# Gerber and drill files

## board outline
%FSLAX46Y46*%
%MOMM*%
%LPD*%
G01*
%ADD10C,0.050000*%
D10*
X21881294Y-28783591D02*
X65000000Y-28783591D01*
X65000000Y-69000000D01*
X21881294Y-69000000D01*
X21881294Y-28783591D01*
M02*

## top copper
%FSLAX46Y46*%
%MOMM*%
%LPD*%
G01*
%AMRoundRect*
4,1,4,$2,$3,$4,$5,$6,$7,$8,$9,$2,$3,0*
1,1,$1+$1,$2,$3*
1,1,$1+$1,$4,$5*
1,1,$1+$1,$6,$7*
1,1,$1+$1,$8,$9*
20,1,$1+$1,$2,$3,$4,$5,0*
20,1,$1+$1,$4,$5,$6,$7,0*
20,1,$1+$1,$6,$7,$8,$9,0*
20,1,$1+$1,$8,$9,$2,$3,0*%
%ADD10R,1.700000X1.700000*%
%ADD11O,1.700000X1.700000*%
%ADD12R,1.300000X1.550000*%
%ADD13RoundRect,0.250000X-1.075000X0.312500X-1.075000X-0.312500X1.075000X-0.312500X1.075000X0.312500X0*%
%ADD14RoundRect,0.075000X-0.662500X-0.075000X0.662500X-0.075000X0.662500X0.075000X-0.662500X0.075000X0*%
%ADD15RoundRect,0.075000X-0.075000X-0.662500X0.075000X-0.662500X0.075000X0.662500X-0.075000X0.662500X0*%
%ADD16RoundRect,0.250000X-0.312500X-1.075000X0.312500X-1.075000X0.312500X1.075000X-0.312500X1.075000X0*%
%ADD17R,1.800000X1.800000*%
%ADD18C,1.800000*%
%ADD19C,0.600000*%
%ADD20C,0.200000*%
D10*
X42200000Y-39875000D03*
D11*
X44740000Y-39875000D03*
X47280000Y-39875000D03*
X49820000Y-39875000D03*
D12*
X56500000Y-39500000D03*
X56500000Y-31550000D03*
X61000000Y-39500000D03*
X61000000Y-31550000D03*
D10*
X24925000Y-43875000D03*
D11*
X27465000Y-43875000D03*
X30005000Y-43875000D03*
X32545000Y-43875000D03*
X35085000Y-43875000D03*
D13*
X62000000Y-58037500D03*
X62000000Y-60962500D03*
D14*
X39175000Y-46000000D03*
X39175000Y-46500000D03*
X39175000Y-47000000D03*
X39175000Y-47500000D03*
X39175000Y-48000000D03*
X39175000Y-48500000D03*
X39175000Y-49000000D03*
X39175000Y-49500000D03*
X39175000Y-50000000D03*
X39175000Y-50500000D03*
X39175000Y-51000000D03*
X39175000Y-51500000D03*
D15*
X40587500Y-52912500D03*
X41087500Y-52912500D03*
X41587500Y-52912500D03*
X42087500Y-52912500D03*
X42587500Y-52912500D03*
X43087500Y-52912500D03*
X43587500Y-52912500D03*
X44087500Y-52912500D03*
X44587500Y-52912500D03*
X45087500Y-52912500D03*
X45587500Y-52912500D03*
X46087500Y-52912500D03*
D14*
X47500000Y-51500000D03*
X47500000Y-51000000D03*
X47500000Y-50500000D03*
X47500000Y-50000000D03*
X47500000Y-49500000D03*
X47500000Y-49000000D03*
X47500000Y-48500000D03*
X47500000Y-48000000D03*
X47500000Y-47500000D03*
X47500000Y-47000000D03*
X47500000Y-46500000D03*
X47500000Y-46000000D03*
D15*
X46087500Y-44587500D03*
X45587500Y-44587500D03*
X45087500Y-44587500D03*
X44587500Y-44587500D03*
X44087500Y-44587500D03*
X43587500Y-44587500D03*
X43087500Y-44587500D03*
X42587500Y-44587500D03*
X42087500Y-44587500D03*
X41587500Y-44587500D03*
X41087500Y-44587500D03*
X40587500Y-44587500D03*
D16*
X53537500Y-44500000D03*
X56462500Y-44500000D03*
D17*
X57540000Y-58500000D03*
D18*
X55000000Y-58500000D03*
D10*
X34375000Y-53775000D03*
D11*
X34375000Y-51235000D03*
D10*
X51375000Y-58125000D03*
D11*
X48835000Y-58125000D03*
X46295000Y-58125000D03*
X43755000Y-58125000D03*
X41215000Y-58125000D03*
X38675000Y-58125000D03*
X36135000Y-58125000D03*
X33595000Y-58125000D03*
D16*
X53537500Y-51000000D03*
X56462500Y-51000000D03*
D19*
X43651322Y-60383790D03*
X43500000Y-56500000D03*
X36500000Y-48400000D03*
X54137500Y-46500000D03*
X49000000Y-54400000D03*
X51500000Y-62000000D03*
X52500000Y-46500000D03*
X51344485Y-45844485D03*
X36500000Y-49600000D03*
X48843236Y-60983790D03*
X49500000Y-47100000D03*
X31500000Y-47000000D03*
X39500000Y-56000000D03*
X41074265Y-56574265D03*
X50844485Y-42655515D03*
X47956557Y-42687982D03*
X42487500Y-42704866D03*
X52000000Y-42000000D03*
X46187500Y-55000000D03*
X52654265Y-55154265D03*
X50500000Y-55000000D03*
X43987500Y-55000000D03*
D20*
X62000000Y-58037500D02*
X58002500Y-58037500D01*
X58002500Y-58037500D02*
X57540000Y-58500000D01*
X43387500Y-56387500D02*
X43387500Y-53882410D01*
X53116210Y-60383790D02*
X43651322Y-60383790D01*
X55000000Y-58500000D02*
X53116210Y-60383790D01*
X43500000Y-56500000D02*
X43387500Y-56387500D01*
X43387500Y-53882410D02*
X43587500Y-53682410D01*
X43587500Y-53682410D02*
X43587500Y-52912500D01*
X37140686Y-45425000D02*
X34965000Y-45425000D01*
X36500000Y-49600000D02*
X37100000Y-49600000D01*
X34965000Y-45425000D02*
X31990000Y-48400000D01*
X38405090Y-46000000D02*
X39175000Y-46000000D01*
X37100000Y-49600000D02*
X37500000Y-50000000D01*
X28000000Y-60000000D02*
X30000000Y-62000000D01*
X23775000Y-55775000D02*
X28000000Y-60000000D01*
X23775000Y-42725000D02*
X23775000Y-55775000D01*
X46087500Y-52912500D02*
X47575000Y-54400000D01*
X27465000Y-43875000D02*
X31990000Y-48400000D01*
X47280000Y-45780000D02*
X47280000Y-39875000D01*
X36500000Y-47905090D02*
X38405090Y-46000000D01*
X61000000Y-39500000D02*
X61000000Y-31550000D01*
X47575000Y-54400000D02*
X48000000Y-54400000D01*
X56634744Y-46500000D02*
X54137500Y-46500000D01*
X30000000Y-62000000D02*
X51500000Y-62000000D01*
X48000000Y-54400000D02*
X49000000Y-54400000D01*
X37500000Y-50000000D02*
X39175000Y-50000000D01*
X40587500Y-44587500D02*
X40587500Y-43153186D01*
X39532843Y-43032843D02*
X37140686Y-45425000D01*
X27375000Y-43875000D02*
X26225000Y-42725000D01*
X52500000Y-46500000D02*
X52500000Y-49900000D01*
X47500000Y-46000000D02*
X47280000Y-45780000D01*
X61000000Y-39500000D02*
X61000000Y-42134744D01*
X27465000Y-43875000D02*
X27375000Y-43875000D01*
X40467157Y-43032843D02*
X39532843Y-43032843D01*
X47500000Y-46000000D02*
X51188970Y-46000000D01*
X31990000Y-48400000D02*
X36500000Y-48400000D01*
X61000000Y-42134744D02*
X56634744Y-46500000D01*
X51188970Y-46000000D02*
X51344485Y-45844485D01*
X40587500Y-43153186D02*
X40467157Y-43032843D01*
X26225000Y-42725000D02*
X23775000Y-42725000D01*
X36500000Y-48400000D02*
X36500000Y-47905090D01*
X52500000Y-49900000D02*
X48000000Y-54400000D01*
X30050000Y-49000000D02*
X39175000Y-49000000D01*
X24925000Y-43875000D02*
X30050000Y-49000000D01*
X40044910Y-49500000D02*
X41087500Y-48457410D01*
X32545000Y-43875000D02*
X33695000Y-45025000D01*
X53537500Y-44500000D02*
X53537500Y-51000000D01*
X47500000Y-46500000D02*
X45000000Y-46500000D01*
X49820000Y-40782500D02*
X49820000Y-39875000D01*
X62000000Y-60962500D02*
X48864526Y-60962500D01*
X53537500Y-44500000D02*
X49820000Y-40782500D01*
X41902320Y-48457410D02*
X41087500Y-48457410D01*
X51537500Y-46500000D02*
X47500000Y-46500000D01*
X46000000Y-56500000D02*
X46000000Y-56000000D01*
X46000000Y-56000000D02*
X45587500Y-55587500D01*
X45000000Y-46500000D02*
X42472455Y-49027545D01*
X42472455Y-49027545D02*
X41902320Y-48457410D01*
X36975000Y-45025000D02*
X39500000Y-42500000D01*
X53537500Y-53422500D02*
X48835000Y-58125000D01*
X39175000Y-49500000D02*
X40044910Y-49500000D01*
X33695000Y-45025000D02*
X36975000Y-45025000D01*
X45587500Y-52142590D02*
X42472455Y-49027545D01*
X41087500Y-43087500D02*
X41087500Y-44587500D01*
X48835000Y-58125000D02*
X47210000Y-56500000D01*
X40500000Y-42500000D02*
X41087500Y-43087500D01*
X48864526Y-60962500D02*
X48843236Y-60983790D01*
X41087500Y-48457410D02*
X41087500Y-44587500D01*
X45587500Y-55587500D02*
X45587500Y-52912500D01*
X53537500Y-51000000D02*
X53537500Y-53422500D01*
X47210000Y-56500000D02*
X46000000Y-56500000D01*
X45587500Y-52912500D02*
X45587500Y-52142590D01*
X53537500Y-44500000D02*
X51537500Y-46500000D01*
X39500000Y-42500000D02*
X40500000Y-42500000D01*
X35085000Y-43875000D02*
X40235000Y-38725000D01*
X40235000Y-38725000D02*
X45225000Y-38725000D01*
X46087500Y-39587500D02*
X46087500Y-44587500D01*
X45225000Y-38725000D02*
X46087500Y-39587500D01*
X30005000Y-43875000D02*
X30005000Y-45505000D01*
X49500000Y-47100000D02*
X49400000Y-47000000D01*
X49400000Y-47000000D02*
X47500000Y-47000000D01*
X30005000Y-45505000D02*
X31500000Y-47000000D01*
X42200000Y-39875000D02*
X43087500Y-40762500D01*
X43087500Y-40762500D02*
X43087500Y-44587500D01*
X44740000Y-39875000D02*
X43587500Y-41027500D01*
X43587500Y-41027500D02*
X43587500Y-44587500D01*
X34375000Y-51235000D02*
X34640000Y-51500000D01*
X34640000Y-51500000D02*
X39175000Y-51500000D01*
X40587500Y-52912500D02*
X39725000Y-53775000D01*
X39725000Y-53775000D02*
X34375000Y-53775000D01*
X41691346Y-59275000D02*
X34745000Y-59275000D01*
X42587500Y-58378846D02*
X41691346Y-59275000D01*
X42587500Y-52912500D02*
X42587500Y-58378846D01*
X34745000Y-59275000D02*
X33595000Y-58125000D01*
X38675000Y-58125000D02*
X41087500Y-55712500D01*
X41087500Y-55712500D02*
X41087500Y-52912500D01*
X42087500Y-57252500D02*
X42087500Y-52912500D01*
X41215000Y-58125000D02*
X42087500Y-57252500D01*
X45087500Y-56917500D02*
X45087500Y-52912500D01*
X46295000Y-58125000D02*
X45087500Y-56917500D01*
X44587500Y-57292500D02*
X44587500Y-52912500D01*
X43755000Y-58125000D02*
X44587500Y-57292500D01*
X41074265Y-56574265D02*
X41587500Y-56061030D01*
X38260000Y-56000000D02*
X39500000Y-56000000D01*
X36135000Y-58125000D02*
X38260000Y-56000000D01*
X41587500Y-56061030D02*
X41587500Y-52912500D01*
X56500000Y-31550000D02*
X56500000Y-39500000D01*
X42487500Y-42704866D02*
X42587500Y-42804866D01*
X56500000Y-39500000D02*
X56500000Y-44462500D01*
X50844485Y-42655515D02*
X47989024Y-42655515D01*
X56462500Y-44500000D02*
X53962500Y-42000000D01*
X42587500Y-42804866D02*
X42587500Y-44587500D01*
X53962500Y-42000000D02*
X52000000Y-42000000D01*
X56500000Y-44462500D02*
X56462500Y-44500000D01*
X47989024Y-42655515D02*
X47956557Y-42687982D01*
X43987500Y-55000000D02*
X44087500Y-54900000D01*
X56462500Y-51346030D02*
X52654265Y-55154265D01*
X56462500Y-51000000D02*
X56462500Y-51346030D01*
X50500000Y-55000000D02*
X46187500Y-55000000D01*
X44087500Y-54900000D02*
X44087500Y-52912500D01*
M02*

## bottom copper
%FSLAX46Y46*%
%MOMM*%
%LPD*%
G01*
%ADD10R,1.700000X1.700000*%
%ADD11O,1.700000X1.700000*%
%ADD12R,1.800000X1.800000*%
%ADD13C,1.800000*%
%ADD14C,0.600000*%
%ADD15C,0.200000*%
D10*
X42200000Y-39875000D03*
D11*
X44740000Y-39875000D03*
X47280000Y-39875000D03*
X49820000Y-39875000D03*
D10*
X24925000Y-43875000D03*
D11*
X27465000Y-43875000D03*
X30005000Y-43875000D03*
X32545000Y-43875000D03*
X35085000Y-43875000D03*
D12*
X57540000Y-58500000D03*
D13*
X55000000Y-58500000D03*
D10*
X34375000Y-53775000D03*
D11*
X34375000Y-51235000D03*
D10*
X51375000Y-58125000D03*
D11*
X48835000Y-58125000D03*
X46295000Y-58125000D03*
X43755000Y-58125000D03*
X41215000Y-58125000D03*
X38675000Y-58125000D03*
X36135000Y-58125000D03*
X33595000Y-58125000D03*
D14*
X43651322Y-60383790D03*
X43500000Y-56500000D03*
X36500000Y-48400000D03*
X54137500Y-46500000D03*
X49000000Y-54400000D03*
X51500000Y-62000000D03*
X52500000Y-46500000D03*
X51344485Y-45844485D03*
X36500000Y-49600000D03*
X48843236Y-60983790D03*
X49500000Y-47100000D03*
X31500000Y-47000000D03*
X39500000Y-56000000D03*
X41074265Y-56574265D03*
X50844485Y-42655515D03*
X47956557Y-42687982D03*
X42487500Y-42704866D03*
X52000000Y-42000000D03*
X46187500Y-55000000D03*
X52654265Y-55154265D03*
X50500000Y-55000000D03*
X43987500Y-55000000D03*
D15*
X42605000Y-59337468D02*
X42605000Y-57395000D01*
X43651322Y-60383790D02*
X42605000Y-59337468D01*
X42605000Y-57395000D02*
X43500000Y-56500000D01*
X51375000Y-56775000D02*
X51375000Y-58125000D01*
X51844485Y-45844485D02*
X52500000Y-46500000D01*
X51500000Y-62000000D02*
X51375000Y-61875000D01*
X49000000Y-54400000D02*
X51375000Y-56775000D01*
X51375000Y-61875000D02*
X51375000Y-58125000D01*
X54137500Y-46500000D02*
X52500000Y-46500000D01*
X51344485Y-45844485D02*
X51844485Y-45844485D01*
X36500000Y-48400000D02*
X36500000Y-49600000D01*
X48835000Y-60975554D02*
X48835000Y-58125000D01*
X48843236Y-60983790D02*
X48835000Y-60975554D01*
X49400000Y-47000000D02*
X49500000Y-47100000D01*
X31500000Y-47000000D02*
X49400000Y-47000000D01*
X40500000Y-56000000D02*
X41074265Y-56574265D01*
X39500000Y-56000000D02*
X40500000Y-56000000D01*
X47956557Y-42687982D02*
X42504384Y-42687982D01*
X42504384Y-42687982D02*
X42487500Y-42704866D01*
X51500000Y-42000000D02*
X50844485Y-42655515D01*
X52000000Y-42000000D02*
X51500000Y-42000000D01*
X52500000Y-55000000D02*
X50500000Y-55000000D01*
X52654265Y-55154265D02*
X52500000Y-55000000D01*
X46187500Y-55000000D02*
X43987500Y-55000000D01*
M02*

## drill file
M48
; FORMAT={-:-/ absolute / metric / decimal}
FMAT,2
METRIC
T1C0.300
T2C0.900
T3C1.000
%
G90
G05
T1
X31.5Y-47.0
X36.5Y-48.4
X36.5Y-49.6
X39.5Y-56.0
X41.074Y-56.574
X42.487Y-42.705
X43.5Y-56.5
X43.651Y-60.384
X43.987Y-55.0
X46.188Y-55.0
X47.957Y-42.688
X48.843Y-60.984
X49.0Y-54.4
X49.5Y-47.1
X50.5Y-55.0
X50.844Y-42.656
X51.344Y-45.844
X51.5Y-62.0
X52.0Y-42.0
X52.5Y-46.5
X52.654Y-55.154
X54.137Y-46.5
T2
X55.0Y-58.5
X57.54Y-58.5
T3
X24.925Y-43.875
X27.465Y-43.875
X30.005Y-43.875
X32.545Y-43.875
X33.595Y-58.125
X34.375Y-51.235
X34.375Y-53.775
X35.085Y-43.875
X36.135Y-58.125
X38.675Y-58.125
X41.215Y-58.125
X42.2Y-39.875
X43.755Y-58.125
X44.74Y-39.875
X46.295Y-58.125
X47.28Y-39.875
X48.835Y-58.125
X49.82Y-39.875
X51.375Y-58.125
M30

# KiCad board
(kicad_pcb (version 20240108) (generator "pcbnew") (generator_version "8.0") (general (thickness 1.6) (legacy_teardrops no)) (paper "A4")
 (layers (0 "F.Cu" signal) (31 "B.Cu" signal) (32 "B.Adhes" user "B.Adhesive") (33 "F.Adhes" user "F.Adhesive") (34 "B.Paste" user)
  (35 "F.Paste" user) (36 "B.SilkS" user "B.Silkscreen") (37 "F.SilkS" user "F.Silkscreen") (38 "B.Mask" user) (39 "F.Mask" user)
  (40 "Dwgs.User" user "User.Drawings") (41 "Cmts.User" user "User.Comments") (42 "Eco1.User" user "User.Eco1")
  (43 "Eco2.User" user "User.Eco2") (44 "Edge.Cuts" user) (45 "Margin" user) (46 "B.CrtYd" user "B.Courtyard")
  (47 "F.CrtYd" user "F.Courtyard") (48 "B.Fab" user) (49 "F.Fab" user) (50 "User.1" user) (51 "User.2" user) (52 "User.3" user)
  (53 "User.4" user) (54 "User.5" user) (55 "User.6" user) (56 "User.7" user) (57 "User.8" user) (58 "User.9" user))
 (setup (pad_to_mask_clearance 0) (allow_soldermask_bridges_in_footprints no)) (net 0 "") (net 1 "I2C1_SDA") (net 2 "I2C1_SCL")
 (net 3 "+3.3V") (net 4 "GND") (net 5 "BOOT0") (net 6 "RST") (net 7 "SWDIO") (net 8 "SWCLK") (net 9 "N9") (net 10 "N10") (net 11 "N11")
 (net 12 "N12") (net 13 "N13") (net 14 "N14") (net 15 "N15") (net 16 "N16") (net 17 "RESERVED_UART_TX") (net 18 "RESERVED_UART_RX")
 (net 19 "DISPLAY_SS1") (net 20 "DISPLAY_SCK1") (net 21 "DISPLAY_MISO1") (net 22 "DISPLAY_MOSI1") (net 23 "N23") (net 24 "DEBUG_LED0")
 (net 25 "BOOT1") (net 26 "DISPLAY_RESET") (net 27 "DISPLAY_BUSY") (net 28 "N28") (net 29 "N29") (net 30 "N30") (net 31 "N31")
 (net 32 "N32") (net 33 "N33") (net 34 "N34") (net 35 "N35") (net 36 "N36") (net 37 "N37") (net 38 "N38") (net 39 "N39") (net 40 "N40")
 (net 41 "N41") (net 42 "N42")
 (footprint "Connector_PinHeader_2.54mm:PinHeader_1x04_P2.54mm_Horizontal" (layer "F.Cu") (at 42.2 39.875 90)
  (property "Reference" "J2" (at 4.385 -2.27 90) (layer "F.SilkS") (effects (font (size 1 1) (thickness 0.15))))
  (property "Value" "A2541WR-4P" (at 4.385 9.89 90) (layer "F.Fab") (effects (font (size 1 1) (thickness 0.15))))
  (pad "1" thru_hole rect (at 0 0 90) (size 1.7 1.7) (drill 1) (layers "*.Cu" "*.Mask") (remove_unused_layers no) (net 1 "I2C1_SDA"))
  (pad "2" thru_hole oval (at 0 2.54 90) (size 1.7 1.7) (drill 1) (layers "*.Cu" "*.Mask") (remove_unused_layers no) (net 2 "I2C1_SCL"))
  (pad "3" thru_hole oval (at 0 5.08 90) (size 1.7 1.7) (drill 1) (layers "*.Cu" "*.Mask") (remove_unused_layers no) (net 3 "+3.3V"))
  (pad "4" thru_hole oval (at 0 7.62 90) (size 1.7 1.7) (drill 1) (layers "*.Cu" "*.Mask") (remove_unused_layers no) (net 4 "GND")))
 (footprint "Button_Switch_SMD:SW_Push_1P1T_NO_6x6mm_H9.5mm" (layer "F.Cu") (at 58.75 35.525 90)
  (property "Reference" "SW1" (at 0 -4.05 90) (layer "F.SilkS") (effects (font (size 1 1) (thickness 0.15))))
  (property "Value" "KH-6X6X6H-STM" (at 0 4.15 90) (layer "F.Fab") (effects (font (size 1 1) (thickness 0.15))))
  (pad "1" smd rect (at -3.975 -2.25 90) (size 1.55 1.3) (layers "F.Cu" "F.Paste" "F.Mask") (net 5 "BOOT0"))
  (pad "1" smd rect (at 3.975 -2.25 90) (size 1.55 1.3) (layers "F.Cu" "F.Paste" "F.Mask") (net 5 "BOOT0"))
  (pad "2" smd rect (at -3.975 2.25 90) (size 1.55 1.3) (layers "F.Cu" "F.Paste" "F.Mask") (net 3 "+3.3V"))
  (pad "2" smd rect (at 3.975 2.25 90) (size 1.55 1.3) (layers "F.Cu" "F.Paste" "F.Mask") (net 3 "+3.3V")))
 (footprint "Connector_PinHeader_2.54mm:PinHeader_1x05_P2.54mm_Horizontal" (layer "F.Cu") (at 24.925 43.875 90)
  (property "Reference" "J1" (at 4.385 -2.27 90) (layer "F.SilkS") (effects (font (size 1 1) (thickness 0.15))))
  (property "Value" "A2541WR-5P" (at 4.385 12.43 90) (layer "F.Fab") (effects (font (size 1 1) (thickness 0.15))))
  (pad "1" thru_hole rect (at 0 0 90) (size 1.7 1.7) (drill 1) (layers "*.Cu" "*.Mask") (remove_unused_layers no) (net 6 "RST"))
  (pad "2" thru_hole oval (at 0 2.54 90) (size 1.7 1.7) (drill 1) (layers "*.Cu" "*.Mask") (remove_unused_layers no) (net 3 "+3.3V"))
  (pad "3" thru_hole oval (at 0 5.08 90) (size 1.7 1.7) (drill 1) (layers "*.Cu" "*.Mask") (remove_unused_layers no) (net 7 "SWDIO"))
  (pad "4" thru_hole oval (at 0 7.62 90) (size 1.7 1.7) (drill 1) (layers "*.Cu" "*.Mask") (remove_unused_layers no) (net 4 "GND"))
  (pad "5" thru_hole oval (at 0 10.16 90) (size 1.7 1.7) (drill 1) (layers "*.Cu" "*.Mask") (remove_unused_layers no) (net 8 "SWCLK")))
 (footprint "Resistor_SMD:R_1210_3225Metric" (layer "F.Cu") (at 62 59.5 -90)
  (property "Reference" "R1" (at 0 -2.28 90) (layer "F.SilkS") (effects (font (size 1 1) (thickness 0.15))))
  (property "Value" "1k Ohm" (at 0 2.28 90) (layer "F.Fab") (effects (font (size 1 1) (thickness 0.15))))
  (pad "1" smd roundrect (at -1.4625 0 270) (size 1.125 2.65) (layers "F.Cu" "F.Paste" "F.Mask") (roundrect_rratio 0.222222) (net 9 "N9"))
  (pad "2" smd roundrect (at 1.4625 0 270) (size 1.125 2.65) (layers "F.Cu" "F.Paste" "F.Mask") (roundrect_rratio 0.222222) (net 4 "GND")))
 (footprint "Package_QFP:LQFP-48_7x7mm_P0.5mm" (layer "F.Cu") (at 43.3375 48.75)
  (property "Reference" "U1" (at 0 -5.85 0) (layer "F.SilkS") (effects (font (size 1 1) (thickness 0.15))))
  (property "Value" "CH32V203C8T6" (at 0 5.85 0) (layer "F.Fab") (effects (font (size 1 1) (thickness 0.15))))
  (pad "1" smd roundrect (at -4.1625 -2.75) (size 1.475 0.3) (layers "F.Cu" "F.Paste" "F.Mask") (roundrect_rratio 0.25) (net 3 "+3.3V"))
  (pad "2" smd roundrect (at -4.1625 -2.25) (size 1.475 0.3) (layers "F.Cu" "F.Paste" "F.Mask") (roundrect_rratio 0.25) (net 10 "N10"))
  (pad "3" smd roundrect (at -4.1625 -1.75) (size 1.475 0.3) (layers "F.Cu" "F.Paste" "F.Mask") (roundrect_rratio 0.25) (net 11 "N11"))
  (pad "4" smd roundrect (at -4.1625 -1.25) (size 1.475 0.3) (layers "F.Cu" "F.Paste" "F.Mask") (roundrect_rratio 0.25) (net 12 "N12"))
  (pad "5" smd roundrect (at -4.1625 -0.75) (size 1.475 0.3) (layers "F.Cu" "F.Paste" "F.Mask") (roundrect_rratio 0.25) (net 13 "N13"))
  (pad "6" smd roundrect (at -4.1625 -0.25) (size 1.475 0.3) (layers "F.Cu" "F.Paste" "F.Mask") (roundrect_rratio 0.25) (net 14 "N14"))
  (pad "7" smd roundrect (at -4.1625 0.25) (size 1.475 0.3) (layers "F.Cu" "F.Paste" "F.Mask") (roundrect_rratio 0.25) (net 6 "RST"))
  (pad "8" smd roundrect (at -4.1625 0.75) (size 1.475 0.3) (layers "F.Cu" "F.Paste" "F.Mask") (roundrect_rratio 0.25) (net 4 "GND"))
  (pad "9" smd roundrect (at -4.1625 1.25) (size 1.475 0.3) (layers "F.Cu" "F.Paste" "F.Mask") (roundrect_rratio 0.25) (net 3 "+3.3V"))
  (pad "10" smd roundrect (at -4.1625 1.75) (size 1.475 0.3) (layers "F.Cu" "F.Paste" "F.Mask") (roundrect_rratio 0.25) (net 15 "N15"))
  (pad "11" smd roundrect (at -4.1625 2.25) (size 1.475 0.3) (layers "F.Cu" "F.Paste" "F.Mask") (roundrect_rratio 0.25) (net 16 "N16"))
  (pad "12" smd roundrect (at -4.1625 2.75) (size 1.475 0.3) (layers "F.Cu" "F.Paste" "F.Mask") (roundrect_rratio 0.25)
   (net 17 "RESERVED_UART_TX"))
  (pad "13" smd roundrect (at -2.75 4.1625) (size 0.3 1.475) (layers "F.Cu" "F.Paste" "F.Mask") (roundrect_rratio 0.25)
   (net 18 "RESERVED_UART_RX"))
  (pad "14" smd roundrect (at -2.25 4.1625) (size 0.3 1.475) (layers "F.Cu" "F.Paste" "F.Mask") (roundrect_rratio 0.25)
   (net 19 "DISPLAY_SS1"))
  (pad "15" smd roundrect (at -1.75 4.1625) (size 0.3 1.475) (layers "F.Cu" "F.Paste" "F.Mask") (roundrect_rratio 0.25)
   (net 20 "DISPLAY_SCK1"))
  (pad "16" smd roundrect (at -1.25 4.1625) (size 0.3 1.475) (layers "F.Cu" "F.Paste" "F.Mask") (roundrect_rratio 0.25)
   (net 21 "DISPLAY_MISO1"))
  (pad "17" smd roundrect (at -0.75 4.1625) (size 0.3 1.475) (layers "F.Cu" "F.Paste" "F.Mask") (roundrect_rratio 0.25)
   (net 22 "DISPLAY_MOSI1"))
  (pad "18" smd roundrect (at -0.25 4.1625) (size 0.3 1.475) (layers "F.Cu" "F.Paste" "F.Mask") (roundrect_rratio 0.25) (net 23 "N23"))
  (pad "19" smd roundrect (at 0.25 4.1625) (size 0.3 1.475) (layers "F.Cu" "F.Paste" "F.Mask") (roundrect_rratio 0.25) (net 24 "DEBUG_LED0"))
  (pad "20" smd roundrect (at 0.75 4.1625) (size 0.3 1.475) (layers "F.Cu" "F.Paste" "F.Mask") (roundrect_rratio 0.25) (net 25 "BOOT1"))
  (pad "21" smd roundrect (at 1.25 4.1625) (size 0.3 1.475) (layers "F.Cu" "F.Paste" "F.Mask") (roundrect_rratio 0.25)
   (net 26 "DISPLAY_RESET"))
  (pad "22" smd roundrect (at 1.75 4.1625) (size 0.3 1.475) (layers "F.Cu" "F.Paste" "F.Mask") (roundrect_rratio 0.25)
   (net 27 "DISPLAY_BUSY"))
  (pad "23" smd roundrect (at 2.25 4.1625) (size 0.3 1.475) (layers "F.Cu" "F.Paste" "F.Mask") (roundrect_rratio 0.25) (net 4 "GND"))
  (pad "24" smd roundrect (at 2.75 4.1625) (size 0.3 1.475) (layers "F.Cu" "F.Paste" "F.Mask") (roundrect_rratio 0.25) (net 3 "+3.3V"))
  (pad "25" smd roundrect (at 4.1625 2.75) (size 1.475 0.3) (layers "F.Cu" "F.Paste" "F.Mask") (roundrect_rratio 0.25) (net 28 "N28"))
  (pad "26" smd roundrect (at 4.1625 2.25) (size 1.475 0.3) (layers "F.Cu" "F.Paste" "F.Mask") (roundrect_rratio 0.25) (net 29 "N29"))
  (pad "27" smd roundrect (at 4.1625 1.75) (size 1.475 0.3) (layers "F.Cu" "F.Paste" "F.Mask") (roundrect_rratio 0.25) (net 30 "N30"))
  (pad "28" smd roundrect (at 4.1625 1.25) (size 1.475 0.3) (layers "F.Cu" "F.Paste" "F.Mask") (roundrect_rratio 0.25) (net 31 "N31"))
  (pad "29" smd roundrect (at 4.1625 0.75) (size 1.475 0.3) (layers "F.Cu" "F.Paste" "F.Mask") (roundrect_rratio 0.25) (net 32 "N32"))
  (pad "30" smd roundrect (at 4.1625 0.25) (size 1.475 0.3) (layers "F.Cu" "F.Paste" "F.Mask") (roundrect_rratio 0.25) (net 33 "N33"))
  (pad "31" smd roundrect (at 4.1625 -0.25) (size 1.475 0.3) (layers "F.Cu" "F.Paste" "F.Mask") (roundrect_rratio 0.25) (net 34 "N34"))
  (pad "32" smd roundrect (at 4.1625 -0.75) (size 1.475 0.3) (layers "F.Cu" "F.Paste" "F.Mask") (roundrect_rratio 0.25) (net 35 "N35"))
  (pad "33" smd roundrect (at 4.1625 -1.25) (size 1.475 0.3) (layers "F.Cu" "F.Paste" "F.Mask") (roundrect_rratio 0.25) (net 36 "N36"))
  (pad "34" smd roundrect (at 4.1625 -1.75) (size 1.475 0.3) (layers "F.Cu" "F.Paste" "F.Mask") (roundrect_rratio 0.25) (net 7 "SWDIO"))
  (pad "35" smd roundrect (at 4.1625 -2.25) (size 1.475 0.3) (layers "F.Cu" "F.Paste" "F.Mask") (roundrect_rratio 0.25) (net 4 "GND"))
  (pad "36" smd roundrect (at 4.1625 -2.75) (size 1.475 0.3) (layers "F.Cu" "F.Paste" "F.Mask") (roundrect_rratio 0.25) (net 3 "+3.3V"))
  (pad "37" smd roundrect (at 2.75 -4.1625) (size 0.3 1.475) (layers "F.Cu" "F.Paste" "F.Mask") (roundrect_rratio 0.25) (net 8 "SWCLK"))
  (pad "38" smd roundrect (at 2.25 -4.1625) (size 0.3 1.475) (layers "F.Cu" "F.Paste" "F.Mask") (roundrect_rratio 0.25) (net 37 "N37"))
  (pad "39" smd roundrect (at 1.75 -4.1625) (size 0.3 1.475) (layers "F.Cu" "F.Paste" "F.Mask") (roundrect_rratio 0.25) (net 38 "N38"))
  (pad "40" smd roundrect (at 1.25 -4.1625) (size 0.3 1.475) (layers "F.Cu" "F.Paste" "F.Mask") (roundrect_rratio 0.25) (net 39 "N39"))
  (pad "41" smd roundrect (at 0.75 -4.1625) (size 0.3 1.475) (layers "F.Cu" "F.Paste" "F.Mask") (roundrect_rratio 0.25) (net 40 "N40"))
  (pad "42" smd roundrect (at 0.25 -4.1625) (size 0.3 1.475) (layers "F.Cu" "F.Paste" "F.Mask") (roundrect_rratio 0.25) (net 2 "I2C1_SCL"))
  (pad "43" smd roundrect (at -0.25 -4.1625) (size 0.3 1.475) (layers "F.Cu" "F.Paste" "F.Mask") (roundrect_rratio 0.25) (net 1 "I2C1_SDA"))
  (pad "44" smd roundrect (at -0.75 -4.1625) (size 0.3 1.475) (layers "F.Cu" "F.Paste" "F.Mask") (roundrect_rratio 0.25) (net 5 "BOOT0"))
  (pad "45" smd roundrect (at -1.25 -4.1625) (size 0.3 1.475) (layers "F.Cu" "F.Paste" "F.Mask") (roundrect_rratio 0.25) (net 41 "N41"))
  (pad "46" smd roundrect (at -1.75 -4.1625) (size 0.3 1.475) (layers "F.Cu" "F.Paste" "F.Mask") (roundrect_rratio 0.25) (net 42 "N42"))
  (pad "47" smd roundrect (at -2.25 -4.1625) (size 0.3 1.475) (layers "F.Cu" "F.Paste" "F.Mask") (roundrect_rratio 0.25) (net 4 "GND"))
  (pad "48" smd roundrect (at -2.75 -4.1625) (size 0.3 1.475) (layers "F.Cu" "F.Paste" "F.Mask") (roundrect_rratio 0.25) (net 3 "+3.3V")))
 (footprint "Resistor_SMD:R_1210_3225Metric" (layer "F.Cu") (at 55 44.5)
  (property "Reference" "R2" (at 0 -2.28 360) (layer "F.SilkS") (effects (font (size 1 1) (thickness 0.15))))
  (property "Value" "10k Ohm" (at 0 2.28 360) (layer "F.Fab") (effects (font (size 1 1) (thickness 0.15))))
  (pad "1" smd roundrect (at -1.4625 0) (size 1.125 2.65) (layers "F.Cu" "F.Paste" "F.Mask") (roundrect_rratio 0.222222) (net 4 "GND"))
  (pad "2" smd roundrect (at 1.4625 0) (size 1.125 2.65) (layers "F.Cu" "F.Paste" "F.Mask") (roundrect_rratio 0.222222) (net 5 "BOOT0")))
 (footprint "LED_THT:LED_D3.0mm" (layer "F.Cu") (at 57.54 58.5 180)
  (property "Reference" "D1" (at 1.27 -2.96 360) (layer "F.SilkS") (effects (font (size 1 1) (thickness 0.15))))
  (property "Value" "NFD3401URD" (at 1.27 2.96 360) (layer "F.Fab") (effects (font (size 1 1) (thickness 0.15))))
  (pad "1" thru_hole rect (at 0 0 180) (size 1.8 1.8) (drill 0.9) (layers "*.Cu" "*.Mask") (remove_unused_layers no) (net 9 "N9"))
  (pad "2" thru_hole circle (at 2.54 0 180) (size 1.8 1.8) (drill 0.9) (layers "*.Cu" "*.Mask") (remove_unused_layers no)
   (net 24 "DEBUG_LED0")))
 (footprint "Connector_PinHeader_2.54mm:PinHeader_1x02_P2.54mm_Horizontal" (layer "F.Cu") (at 34.375 53.775 180)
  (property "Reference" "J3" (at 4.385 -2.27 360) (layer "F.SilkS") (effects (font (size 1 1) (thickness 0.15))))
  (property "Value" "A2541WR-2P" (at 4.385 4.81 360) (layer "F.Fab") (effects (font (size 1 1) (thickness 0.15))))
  (pad "1" thru_hole rect (at 0 0 180) (size 1.7 1.7) (drill 1) (layers "*.Cu" "*.Mask") (remove_unused_layers no)
   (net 18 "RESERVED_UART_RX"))
  (pad "2" thru_hole oval (at 0 2.54 180) (size 1.7 1.7) (drill 1) (layers "*.Cu" "*.Mask") (remove_unused_layers no)
   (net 17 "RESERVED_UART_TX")))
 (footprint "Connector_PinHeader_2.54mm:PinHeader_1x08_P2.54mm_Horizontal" (layer "F.Cu") (at 51.375 58.125 -90)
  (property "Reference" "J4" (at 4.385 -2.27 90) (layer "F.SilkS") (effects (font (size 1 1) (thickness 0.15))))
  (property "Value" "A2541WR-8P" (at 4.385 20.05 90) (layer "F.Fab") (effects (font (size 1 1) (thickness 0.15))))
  (pad "1" thru_hole rect (at 0 0 270) (size 1.7 1.7) (drill 1) (layers "*.Cu" "*.Mask") (remove_unused_layers no) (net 3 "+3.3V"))
  (pad "2" thru_hole oval (at 0 2.54 270) (size 1.7 1.7) (drill 1) (layers "*.Cu" "*.Mask") (remove_unused_layers no) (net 4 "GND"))
  (pad "3" thru_hole oval (at 0 5.08 270) (size 1.7 1.7) (drill 1) (layers "*.Cu" "*.Mask") (remove_unused_layers no)
   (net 27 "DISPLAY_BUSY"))
  (pad "4" thru_hole oval (at 0 7.62 270) (size 1.7 1.7) (drill 1) (layers "*.Cu" "*.Mask") (remove_unused_layers no)
   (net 26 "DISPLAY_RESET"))
  (pad "5" thru_hole oval (at 0 10.16 270) (size 1.7 1.7) (drill 1) (layers "*.Cu" "*.Mask") (remove_unused_layers no)
   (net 21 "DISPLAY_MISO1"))
  (pad "6" thru_hole oval (at 0 12.7 270) (size 1.7 1.7) (drill 1) (layers "*.Cu" "*.Mask") (remove_unused_layers no) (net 19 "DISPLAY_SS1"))
  (pad "7" thru_hole oval (at 0 15.24 270) (size 1.7 1.7) (drill 1) (layers "*.Cu" "*.Mask") (remove_unused_layers no)
   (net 20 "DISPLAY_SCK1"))
  (pad "8" thru_hole oval (at 0 17.78 270) (size 1.7 1.7) (drill 1) (layers "*.Cu" "*.Mask") (remove_unused_layers no)
   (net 22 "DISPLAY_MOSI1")))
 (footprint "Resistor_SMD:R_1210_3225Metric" (layer "F.Cu") (at 55 51)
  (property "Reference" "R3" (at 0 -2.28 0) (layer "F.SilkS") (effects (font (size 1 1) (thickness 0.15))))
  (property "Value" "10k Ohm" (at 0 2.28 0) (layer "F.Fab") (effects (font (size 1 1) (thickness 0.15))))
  (pad "1" smd roundrect (at -1.4625 0) (size 1.125 2.65) (layers "F.Cu" "F.Paste" "F.Mask") (roundrect_rratio 0.222222) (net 4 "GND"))
  (pad "2" smd roundrect (at 1.4625 0) (size 1.125 2.65) (layers "F.Cu" "F.Paste" "F.Mask") (roundrect_rratio 0.222222) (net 25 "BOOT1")))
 (gr_rect (start 21.881294 28.783591) (end 65 69) (stroke (width 0.05) (type default)) (fill none) (layer "Edge.Cuts"))
 (segment (start 62 58.0375) (end 58.0025 58.0375) (width 0.2) (layer "F.Cu") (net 9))
 (segment (start 58.0025 58.0375) (end 57.54 58.5) (width 0.2) (layer "F.Cu") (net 9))
 (segment (start 43.3875 56.3875) (end 43.3875 53.88241) (width 0.2) (layer "F.Cu") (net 24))
 (segment (start 53.11621 60.38379) (end 43.651322 60.38379) (width 0.2) (layer "F.Cu") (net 24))
 (segment (start 55 58.5) (end 53.11621 60.38379) (width 0.2) (layer "F.Cu") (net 24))
 (segment (start 43.5 56.5) (end 43.3875 56.3875) (width 0.2) (layer "F.Cu") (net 24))
 (segment (start 43.3875 53.88241) (end 43.5875 53.68241) (width 0.2) (layer "F.Cu") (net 24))
 (segment (start 43.5875 53.68241) (end 43.5875 52.9125) (width 0.2) (layer "F.Cu") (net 24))
 (via (at 43.651322 60.38379) (size 0.6) (drill 0.3) (layers "F.Cu" "B.Cu") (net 24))
 (via (at 43.5 56.5) (size 0.6) (drill 0.3) (layers "F.Cu" "B.Cu") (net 24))
 (segment (start 42.605 59.337468) (end 42.605 57.395) (width 0.2) (layer "B.Cu") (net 24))
 (segment (start 43.651322 60.38379) (end 42.605 59.337468) (width 0.2) (layer "B.Cu") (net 24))
 (segment (start 42.605 57.395) (end 43.5 56.5) (width 0.2) (layer "B.Cu") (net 24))
 (segment (start 37.140686 45.425) (end 34.965 45.425) (width 0.2) (layer "F.Cu") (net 3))
 (segment (start 36.5 49.6) (end 37.1 49.6) (width 0.2) (layer "F.Cu") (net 3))
 (segment (start 34.965 45.425) (end 31.99 48.4) (width 0.2) (layer "F.Cu") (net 3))
 (segment (start 38.40509 46) (end 39.175 46) (width 0.2) (layer "F.Cu") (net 3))
 (segment (start 37.1 49.6) (end 37.5 50) (width 0.2) (layer "F.Cu") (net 3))
 (segment (start 28 60) (end 30 62) (width 0.2) (layer "F.Cu") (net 3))
 (segment (start 23.775 55.775) (end 28 60) (width 0.2) (layer "F.Cu") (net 3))
 (segment (start 23.775 42.725) (end 23.775 55.775) (width 0.2) (layer "F.Cu") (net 3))
 (segment (start 46.0875 52.9125) (end 47.575 54.4) (width 0.2) (layer "F.Cu") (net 3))
 (segment (start 27.465 43.875) (end 31.99 48.4) (width 0.2) (layer "F.Cu") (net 3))
 (segment (start 47.28 45.78) (end 47.28 39.875) (width 0.2) (layer "F.Cu") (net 3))
 (segment (start 36.5 47.90509) (end 38.40509 46) (width 0.2) (layer "F.Cu") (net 3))
 (segment (start 61 39.5) (end 61 31.55) (width 0.2) (layer "F.Cu") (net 3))
 (segment (start 47.575 54.4) (end 48 54.4) (width 0.2) (layer "F.Cu") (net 3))
 (segment (start 56.634744 46.5) (end 54.1375 46.5) (width 0.2) (layer "F.Cu") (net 3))
 (segment (start 30 62) (end 51.5 62) (width 0.2) (layer "F.Cu") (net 3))
 (segment (start 48 54.4) (end 49 54.4) (width 0.2) (layer "F.Cu") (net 3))
 (segment (start 37.5 50) (end 39.175 50) (width 0.2) (layer "F.Cu") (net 3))
 (segment (start 40.5875 44.5875) (end 40.5875 43.153186) (width 0.2) (layer "F.Cu") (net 3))
 (segment (start 39.532843 43.032843) (end 37.140686 45.425) (width 0.2) (layer "F.Cu") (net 3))
 (segment (start 27.375 43.875) (end 26.225 42.725) (width 0.2) (layer "F.Cu") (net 3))
 (segment (start 52.5 46.5) (end 52.5 49.9) (width 0.2) (layer "F.Cu") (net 3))
 (segment (start 47.5 46) (end 47.28 45.78) (width 0.2) (layer "F.Cu") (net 3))
 (segment (start 61 39.5) (end 61 42.134744) (width 0.2) (layer "F.Cu") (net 3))
 (segment (start 27.465 43.875) (end 27.375 43.875) (width 0.2) (layer "F.Cu") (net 3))
 (segment (start 40.467157 43.032843) (end 39.532843 43.032843) (width 0.2) (layer "F.Cu") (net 3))
 (segment (start 47.5 46) (end 51.18897 46) (width 0.2) (layer "F.Cu") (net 3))
 (segment (start 31.99 48.4) (end 36.5 48.4) (width 0.2) (layer "F.Cu") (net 3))
 (segment (start 61 42.134744) (end 56.634744 46.5) (width 0.2) (layer "F.Cu") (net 3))
 (segment (start 51.18897 46) (end 51.344485 45.844485) (width 0.2) (layer "F.Cu") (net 3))
 (segment (start 40.5875 43.153186) (end 40.467157 43.032843) (width 0.2) (layer "F.Cu") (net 3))
 (segment (start 26.225 42.725) (end 23.775 42.725) (width 0.2) (layer "F.Cu") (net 3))
 (segment (start 36.5 48.4) (end 36.5 47.90509) (width 0.2) (layer "F.Cu") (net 3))
 (segment (start 52.5 49.9) (end 48 54.4) (width 0.2) (layer "F.Cu") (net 3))
 (via (at 36.5 48.4) (size 0.6) (drill 0.3) (layers "F.Cu" "B.Cu") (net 3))
 (via (at 54.1375 46.5) (size 0.6) (drill 0.3) (layers "F.Cu" "B.Cu") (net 3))
 (via (at 49 54.4) (size 0.6) (drill 0.3) (layers "F.Cu" "B.Cu") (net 3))
 (via (at 51.5 62) (size 0.6) (drill 0.3) (layers "F.Cu" "B.Cu") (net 3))
 (via (at 52.5 46.5) (size 0.6) (drill 0.3) (layers "F.Cu" "B.Cu") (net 3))
 (via (at 51.344485 45.844485) (size 0.6) (drill 0.3) (layers "F.Cu" "B.Cu") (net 3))
 (via (at 36.5 49.6) (size 0.6) (drill 0.3) (layers "F.Cu" "B.Cu") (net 3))
 (segment (start 51.375 56.775) (end 51.375 58.125) (width 0.2) (layer "B.Cu") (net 3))
 (segment (start 51.844485 45.844485) (end 52.5 46.5) (width 0.2) (layer "B.Cu") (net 3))
 (segment (start 51.5 62) (end 51.375 61.875) (width 0.2) (layer "B.Cu") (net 3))
 (segment (start 49 54.4) (end 51.375 56.775) (width 0.2) (layer "B.Cu") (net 3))
 (segment (start 51.375 61.875) (end 51.375 58.125) (width 0.2) (layer "B.Cu") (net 3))
 (segment (start 54.1375 46.5) (end 52.5 46.5) (width 0.2) (layer "B.Cu") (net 3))
 (segment (start 51.344485 45.844485) (end 51.844485 45.844485) (width 0.2) (layer "B.Cu") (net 3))
 (segment (start 36.5 48.4) (end 36.5 49.6) (width 0.2) (layer "B.Cu") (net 3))
 (segment (start 30.05 49) (end 39.175 49) (width 0.2) (layer "F.Cu") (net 6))
 (segment (start 24.925 43.875) (end 30.05 49) (width 0.2) (layer "F.Cu") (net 6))
 (segment (start 40.04491 49.5) (end 41.0875 48.45741) (width 0.2) (layer "F.Cu") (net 4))
 (segment (start 32.545 43.875) (end 33.695 45.025) (width 0.2) (layer "F.Cu") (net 4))
 (segment (start 53.5375 44.5) (end 53.5375 51) (width 0.2) (layer "F.Cu") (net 4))
 (segment (start 47.5 46.5) (end 45 46.5) (width 0.2) (layer "F.Cu") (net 4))
 (segment (start 49.82 40.7825) (end 49.82 39.875) (width 0.2) (layer "F.Cu") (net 4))
 (segment (start 62 60.9625) (end 48.864526 60.9625) (width 0.2) (layer "F.Cu") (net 4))
 (segment (start 53.5375 44.5) (end 49.82 40.7825) (width 0.2) (layer "F.Cu") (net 4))
 (segment (start 41.90232 48.45741) (end 41.0875 48.45741) (width 0.2) (layer "F.Cu") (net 4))
 (segment (start 51.5375 46.5) (end 47.5 46.5) (width 0.2) (layer "F.Cu") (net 4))
 (segment (start 46 56.5) (end 46 56) (width 0.2) (layer "F.Cu") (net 4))
 (segment (start 46 56) (end 45.5875 55.5875) (width 0.2) (layer "F.Cu") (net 4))
 (segment (start 45 46.5) (end 42.472455 49.027545) (width 0.2) (layer "F.Cu") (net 4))
 (segment (start 42.472455 49.027545) (end 41.90232 48.45741) (width 0.2) (layer "F.Cu") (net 4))
 (segment (start 36.975 45.025) (end 39.5 42.5) (width 0.2) (layer "F.Cu") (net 4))
 (segment (start 53.5375 53.4225) (end 48.835 58.125) (width 0.2) (layer "F.Cu") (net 4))
 (segment (start 39.175 49.5) (end 40.04491 49.5) (width 0.2) (layer "F.Cu") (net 4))
 (segment (start 33.695 45.025) (end 36.975 45.025) (width 0.2) (layer "F.Cu") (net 4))
 (segment (start 45.5875 52.14259) (end 42.472455 49.027545) (width 0.2) (layer "F.Cu") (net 4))
 (segment (start 41.0875 43.0875) (end 41.0875 44.5875) (width 0.2) (layer "F.Cu") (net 4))
 (segment (start 48.835 58.125) (end 47.21 56.5) (width 0.2) (layer "F.Cu") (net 4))
 (segment (start 40.5 42.5) (end 41.0875 43.0875) (width 0.2) (layer "F.Cu") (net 4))
 (segment (start 48.864526 60.9625) (end 48.843236 60.98379) (width 0.2) (layer "F.Cu") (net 4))
 (segment (start 41.0875 48.45741) (end 41.0875 44.5875) (width 0.2) (layer "F.Cu") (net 4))
 (segment (start 45.5875 55.5875) (end 45.5875 52.9125) (width 0.2) (layer "F.Cu") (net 4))
 (segment (start 53.5375 51) (end 53.5375 53.4225) (width 0.2) (layer "F.Cu") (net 4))
 (segment (start 47.21 56.5) (end 46 56.5) (width 0.2) (layer "F.Cu") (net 4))
 (segment (start 45.5875 52.9125) (end 45.5875 52.14259) (width 0.2) (layer "F.Cu") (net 4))
 (segment (start 53.5375 44.5) (end 51.5375 46.5) (width 0.2) (layer "F.Cu") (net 4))
 (segment (start 39.5 42.5) (end 40.5 42.5) (width 0.2) (layer "F.Cu") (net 4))
 (via (at 48.843236 60.98379) (size 0.6) (drill 0.3) (layers "F.Cu" "B.Cu") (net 4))
 (segment (start 48.835 60.975554) (end 48.835 58.125) (width 0.2) (layer "B.Cu") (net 4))
 (segment (start 48.843236 60.98379) (end 48.835 60.975554) (width 0.2) (layer "B.Cu") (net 4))
 (segment (start 35.085 43.875) (end 40.235 38.725) (width 0.2) (layer "F.Cu") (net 8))
 (segment (start 40.235 38.725) (end 45.225 38.725) (width 0.2) (layer "F.Cu") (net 8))
 (segment (start 46.0875 39.5875) (end 46.0875 44.5875) (width 0.2) (layer "F.Cu") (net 8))
 (segment (start 45.225 38.725) (end 46.0875 39.5875) (width 0.2) (layer "F.Cu") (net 8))
 (segment (start 30.005 43.875) (end 30.005 45.505) (width 0.2) (layer "F.Cu") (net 7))
 (segment (start 49.5 47.1) (end 49.4 47) (width 0.2) (layer "F.Cu") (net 7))
 (segment (start 49.4 47) (end 47.5 47) (width 0.2) (layer "F.Cu") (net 7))
 (segment (start 30.005 45.505) (end 31.5 47) (width 0.2) (layer "F.Cu") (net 7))
 (via (at 49.5 47.1) (size 0.6) (drill 0.3) (layers "F.Cu" "B.Cu") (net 7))
 (via (at 31.5 47) (size 0.6) (drill 0.3) (layers "F.Cu" "B.Cu") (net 7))
 (segment (start 49.4 47) (end 49.5 47.1) (width 0.2) (layer "B.Cu") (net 7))
 (segment (start 31.5 47) (end 49.4 47) (width 0.2) (layer "B.Cu") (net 7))
 (segment (start 42.2 39.875) (end 43.0875 40.7625) (width 0.2) (layer "F.Cu") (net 1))
 (segment (start 43.0875 40.7625) (end 43.0875 44.5875) (width 0.2) (layer "F.Cu") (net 1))
 (segment (start 44.74 39.875) (end 43.5875 41.0275) (width 0.2) (layer "F.Cu") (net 2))
 (segment (start 43.5875 41.0275) (end 43.5875 44.5875) (width 0.2) (layer "F.Cu") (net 2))
 (segment (start 34.375 51.235) (end 34.64 51.5) (width 0.2) (layer "F.Cu") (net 17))
 (segment (start 34.64 51.5) (end 39.175 51.5) (width 0.2) (layer "F.Cu") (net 17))
 (segment (start 40.5875 52.9125) (end 39.725 53.775) (width 0.2) (layer "F.Cu") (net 18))
 (segment (start 39.725 53.775) (end 34.375 53.775) (width 0.2) (layer "F.Cu") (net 18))
 (segment (start 41.691346 59.275) (end 34.745 59.275) (width 0.2) (layer "F.Cu") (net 22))
 (segment (start 42.5875 58.378846) (end 41.691346 59.275) (width 0.2) (layer "F.Cu") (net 22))
 (segment (start 42.5875 52.9125) (end 42.5875 58.378846) (width 0.2) (layer "F.Cu") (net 22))
 (segment (start 34.745 59.275) (end 33.595 58.125) (width 0.2) (layer "F.Cu") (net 22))
 (segment (start 38.675 58.125) (end 41.0875 55.7125) (width 0.2) (layer "F.Cu") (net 19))
 (segment (start 41.0875 55.7125) (end 41.0875 52.9125) (width 0.2) (layer "F.Cu") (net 19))
 (segment (start 42.0875 57.2525) (end 42.0875 52.9125) (width 0.2) (layer "F.Cu") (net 21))
 (segment (start 41.215 58.125) (end 42.0875 57.2525) (width 0.2) (layer "F.Cu") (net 21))
 (segment (start 45.0875 56.9175) (end 45.0875 52.9125) (width 0.2) (layer "F.Cu") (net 27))
 (segment (start 46.295 58.125) (end 45.0875 56.9175) (width 0.2) (layer "F.Cu") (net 27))
 (segment (start 44.5875 57.2925) (end 44.5875 52.9125) (width 0.2) (layer "F.Cu") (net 26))
 (segment (start 43.755 58.125) (end 44.5875 57.2925) (width 0.2) (layer "F.Cu") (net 26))
 (segment (start 41.074265 56.574265) (end 41.5875 56.06103) (width 0.2) (layer "F.Cu") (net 20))
 (segment (start 38.26 56) (end 39.5 56) (width 0.2) (layer "F.Cu") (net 20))
 (segment (start 36.135 58.125) (end 38.26 56) (width 0.2) (layer "F.Cu") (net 20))
 (segment (start 41.5875 56.06103) (end 41.5875 52.9125) (width 0.2) (layer "F.Cu") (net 20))
 (via (at 39.5 56) (size 0.6) (drill 0.3) (layers "F.Cu" "B.Cu") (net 20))
 (via (at 41.074265 56.574265) (size 0.6) (drill 0.3) (layers "F.Cu" "B.Cu") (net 20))
 (segment (start 40.5 56) (end 41.074265 56.574265) (width 0.2) (layer "B.Cu") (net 20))
 (segment (start 39.5 56) (end 40.5 56) (width 0.2) (layer "B.Cu") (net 20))
 (segment (start 56.5 31.55) (end 56.5 39.5) (width 0.2) (layer "F.Cu") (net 5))
 (segment (start 42.4875 42.704866) (end 42.5875 42.804866) (width 0.2) (layer "F.Cu") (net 5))
 (segment (start 56.5 39.5) (end 56.5 44.4625) (width 0.2) (layer "F.Cu") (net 5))
 (segment (start 50.844485 42.655515) (end 47.989024 42.655515) (width 0.2) (layer "F.Cu") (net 5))
 (segment (start 56.4625 44.5) (end 53.9625 42) (width 0.2) (layer "F.Cu") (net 5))
 (segment (start 42.5875 42.804866) (end 42.5875 44.5875) (width 0.2) (layer "F.Cu") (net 5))
 (segment (start 53.9625 42) (end 52 42) (width 0.2) (layer "F.Cu") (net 5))
 (segment (start 56.5 44.4625) (end 56.4625 44.5) (width 0.2) (layer "F.Cu") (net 5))
 (segment (start 47.989024 42.655515) (end 47.956557 42.687982) (width 0.2) (layer "F.Cu") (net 5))
 (via (at 50.844485 42.655515) (size 0.6) (drill 0.3) (layers "F.Cu" "B.Cu") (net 5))
 (via (at 47.956557 42.687982) (size 0.6) (drill 0.3) (layers "F.Cu" "B.Cu") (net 5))
 (via (at 42.4875 42.704866) (size 0.6) (drill 0.3) (layers "F.Cu" "B.Cu") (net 5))
 (via (at 52 42) (size 0.6) (drill 0.3) (layers "F.Cu" "B.Cu") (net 5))
 (segment (start 47.956557 42.687982) (end 42.504384 42.687982) (width 0.2) (layer "B.Cu") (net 5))
 (segment (start 42.504384 42.687982) (end 42.4875 42.704866) (width 0.2) (layer "B.Cu") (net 5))
 (segment (start 51.5 42) (end 50.844485 42.655515) (width 0.2) (layer "B.Cu") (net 5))
 (segment (start 52 42) (end 51.5 42) (width 0.2) (layer "B.Cu") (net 5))
 (segment (start 43.9875 55) (end 44.0875 54.9) (width 0.2) (layer "F.Cu") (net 25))
 (segment (start 56.4625 51.34603) (end 52.654265 55.154265) (width 0.2) (layer "F.Cu") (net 25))
 (segment (start 56.4625 51) (end 56.4625 51.34603) (width 0.2) (layer "F.Cu") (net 25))
 (segment (start 50.5 55) (end 46.1875 55) (width 0.2) (layer "F.Cu") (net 25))
 (segment (start 44.0875 54.9) (end 44.0875 52.9125) (width 0.2) (layer "F.Cu") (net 25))
 (via (at 46.1875 55) (size 0.6) (drill 0.3) (layers "F.Cu" "B.Cu") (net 25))
 (via (at 52.654265 55.154265) (size 0.6) (drill 0.3) (layers "F.Cu" "B.Cu") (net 25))
 (via (at 50.5 55) (size 0.6) (drill 0.3) (layers "F.Cu" "B.Cu") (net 25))
 (via (at 43.9875 55) (size 0.6) (drill 0.3) (layers "F.Cu" "B.Cu") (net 25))
 (segment (start 52.5 55) (end 50.5 55) (width 0.2) (layer "B.Cu") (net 25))
 (segment (start 52.654265 55.154265) (end 52.5 55) (width 0.2) (layer "B.Cu") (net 25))
 (segment (start 46.1875 55) (end 43.9875 55) (width 0.2) (layer "B.Cu") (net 25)))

